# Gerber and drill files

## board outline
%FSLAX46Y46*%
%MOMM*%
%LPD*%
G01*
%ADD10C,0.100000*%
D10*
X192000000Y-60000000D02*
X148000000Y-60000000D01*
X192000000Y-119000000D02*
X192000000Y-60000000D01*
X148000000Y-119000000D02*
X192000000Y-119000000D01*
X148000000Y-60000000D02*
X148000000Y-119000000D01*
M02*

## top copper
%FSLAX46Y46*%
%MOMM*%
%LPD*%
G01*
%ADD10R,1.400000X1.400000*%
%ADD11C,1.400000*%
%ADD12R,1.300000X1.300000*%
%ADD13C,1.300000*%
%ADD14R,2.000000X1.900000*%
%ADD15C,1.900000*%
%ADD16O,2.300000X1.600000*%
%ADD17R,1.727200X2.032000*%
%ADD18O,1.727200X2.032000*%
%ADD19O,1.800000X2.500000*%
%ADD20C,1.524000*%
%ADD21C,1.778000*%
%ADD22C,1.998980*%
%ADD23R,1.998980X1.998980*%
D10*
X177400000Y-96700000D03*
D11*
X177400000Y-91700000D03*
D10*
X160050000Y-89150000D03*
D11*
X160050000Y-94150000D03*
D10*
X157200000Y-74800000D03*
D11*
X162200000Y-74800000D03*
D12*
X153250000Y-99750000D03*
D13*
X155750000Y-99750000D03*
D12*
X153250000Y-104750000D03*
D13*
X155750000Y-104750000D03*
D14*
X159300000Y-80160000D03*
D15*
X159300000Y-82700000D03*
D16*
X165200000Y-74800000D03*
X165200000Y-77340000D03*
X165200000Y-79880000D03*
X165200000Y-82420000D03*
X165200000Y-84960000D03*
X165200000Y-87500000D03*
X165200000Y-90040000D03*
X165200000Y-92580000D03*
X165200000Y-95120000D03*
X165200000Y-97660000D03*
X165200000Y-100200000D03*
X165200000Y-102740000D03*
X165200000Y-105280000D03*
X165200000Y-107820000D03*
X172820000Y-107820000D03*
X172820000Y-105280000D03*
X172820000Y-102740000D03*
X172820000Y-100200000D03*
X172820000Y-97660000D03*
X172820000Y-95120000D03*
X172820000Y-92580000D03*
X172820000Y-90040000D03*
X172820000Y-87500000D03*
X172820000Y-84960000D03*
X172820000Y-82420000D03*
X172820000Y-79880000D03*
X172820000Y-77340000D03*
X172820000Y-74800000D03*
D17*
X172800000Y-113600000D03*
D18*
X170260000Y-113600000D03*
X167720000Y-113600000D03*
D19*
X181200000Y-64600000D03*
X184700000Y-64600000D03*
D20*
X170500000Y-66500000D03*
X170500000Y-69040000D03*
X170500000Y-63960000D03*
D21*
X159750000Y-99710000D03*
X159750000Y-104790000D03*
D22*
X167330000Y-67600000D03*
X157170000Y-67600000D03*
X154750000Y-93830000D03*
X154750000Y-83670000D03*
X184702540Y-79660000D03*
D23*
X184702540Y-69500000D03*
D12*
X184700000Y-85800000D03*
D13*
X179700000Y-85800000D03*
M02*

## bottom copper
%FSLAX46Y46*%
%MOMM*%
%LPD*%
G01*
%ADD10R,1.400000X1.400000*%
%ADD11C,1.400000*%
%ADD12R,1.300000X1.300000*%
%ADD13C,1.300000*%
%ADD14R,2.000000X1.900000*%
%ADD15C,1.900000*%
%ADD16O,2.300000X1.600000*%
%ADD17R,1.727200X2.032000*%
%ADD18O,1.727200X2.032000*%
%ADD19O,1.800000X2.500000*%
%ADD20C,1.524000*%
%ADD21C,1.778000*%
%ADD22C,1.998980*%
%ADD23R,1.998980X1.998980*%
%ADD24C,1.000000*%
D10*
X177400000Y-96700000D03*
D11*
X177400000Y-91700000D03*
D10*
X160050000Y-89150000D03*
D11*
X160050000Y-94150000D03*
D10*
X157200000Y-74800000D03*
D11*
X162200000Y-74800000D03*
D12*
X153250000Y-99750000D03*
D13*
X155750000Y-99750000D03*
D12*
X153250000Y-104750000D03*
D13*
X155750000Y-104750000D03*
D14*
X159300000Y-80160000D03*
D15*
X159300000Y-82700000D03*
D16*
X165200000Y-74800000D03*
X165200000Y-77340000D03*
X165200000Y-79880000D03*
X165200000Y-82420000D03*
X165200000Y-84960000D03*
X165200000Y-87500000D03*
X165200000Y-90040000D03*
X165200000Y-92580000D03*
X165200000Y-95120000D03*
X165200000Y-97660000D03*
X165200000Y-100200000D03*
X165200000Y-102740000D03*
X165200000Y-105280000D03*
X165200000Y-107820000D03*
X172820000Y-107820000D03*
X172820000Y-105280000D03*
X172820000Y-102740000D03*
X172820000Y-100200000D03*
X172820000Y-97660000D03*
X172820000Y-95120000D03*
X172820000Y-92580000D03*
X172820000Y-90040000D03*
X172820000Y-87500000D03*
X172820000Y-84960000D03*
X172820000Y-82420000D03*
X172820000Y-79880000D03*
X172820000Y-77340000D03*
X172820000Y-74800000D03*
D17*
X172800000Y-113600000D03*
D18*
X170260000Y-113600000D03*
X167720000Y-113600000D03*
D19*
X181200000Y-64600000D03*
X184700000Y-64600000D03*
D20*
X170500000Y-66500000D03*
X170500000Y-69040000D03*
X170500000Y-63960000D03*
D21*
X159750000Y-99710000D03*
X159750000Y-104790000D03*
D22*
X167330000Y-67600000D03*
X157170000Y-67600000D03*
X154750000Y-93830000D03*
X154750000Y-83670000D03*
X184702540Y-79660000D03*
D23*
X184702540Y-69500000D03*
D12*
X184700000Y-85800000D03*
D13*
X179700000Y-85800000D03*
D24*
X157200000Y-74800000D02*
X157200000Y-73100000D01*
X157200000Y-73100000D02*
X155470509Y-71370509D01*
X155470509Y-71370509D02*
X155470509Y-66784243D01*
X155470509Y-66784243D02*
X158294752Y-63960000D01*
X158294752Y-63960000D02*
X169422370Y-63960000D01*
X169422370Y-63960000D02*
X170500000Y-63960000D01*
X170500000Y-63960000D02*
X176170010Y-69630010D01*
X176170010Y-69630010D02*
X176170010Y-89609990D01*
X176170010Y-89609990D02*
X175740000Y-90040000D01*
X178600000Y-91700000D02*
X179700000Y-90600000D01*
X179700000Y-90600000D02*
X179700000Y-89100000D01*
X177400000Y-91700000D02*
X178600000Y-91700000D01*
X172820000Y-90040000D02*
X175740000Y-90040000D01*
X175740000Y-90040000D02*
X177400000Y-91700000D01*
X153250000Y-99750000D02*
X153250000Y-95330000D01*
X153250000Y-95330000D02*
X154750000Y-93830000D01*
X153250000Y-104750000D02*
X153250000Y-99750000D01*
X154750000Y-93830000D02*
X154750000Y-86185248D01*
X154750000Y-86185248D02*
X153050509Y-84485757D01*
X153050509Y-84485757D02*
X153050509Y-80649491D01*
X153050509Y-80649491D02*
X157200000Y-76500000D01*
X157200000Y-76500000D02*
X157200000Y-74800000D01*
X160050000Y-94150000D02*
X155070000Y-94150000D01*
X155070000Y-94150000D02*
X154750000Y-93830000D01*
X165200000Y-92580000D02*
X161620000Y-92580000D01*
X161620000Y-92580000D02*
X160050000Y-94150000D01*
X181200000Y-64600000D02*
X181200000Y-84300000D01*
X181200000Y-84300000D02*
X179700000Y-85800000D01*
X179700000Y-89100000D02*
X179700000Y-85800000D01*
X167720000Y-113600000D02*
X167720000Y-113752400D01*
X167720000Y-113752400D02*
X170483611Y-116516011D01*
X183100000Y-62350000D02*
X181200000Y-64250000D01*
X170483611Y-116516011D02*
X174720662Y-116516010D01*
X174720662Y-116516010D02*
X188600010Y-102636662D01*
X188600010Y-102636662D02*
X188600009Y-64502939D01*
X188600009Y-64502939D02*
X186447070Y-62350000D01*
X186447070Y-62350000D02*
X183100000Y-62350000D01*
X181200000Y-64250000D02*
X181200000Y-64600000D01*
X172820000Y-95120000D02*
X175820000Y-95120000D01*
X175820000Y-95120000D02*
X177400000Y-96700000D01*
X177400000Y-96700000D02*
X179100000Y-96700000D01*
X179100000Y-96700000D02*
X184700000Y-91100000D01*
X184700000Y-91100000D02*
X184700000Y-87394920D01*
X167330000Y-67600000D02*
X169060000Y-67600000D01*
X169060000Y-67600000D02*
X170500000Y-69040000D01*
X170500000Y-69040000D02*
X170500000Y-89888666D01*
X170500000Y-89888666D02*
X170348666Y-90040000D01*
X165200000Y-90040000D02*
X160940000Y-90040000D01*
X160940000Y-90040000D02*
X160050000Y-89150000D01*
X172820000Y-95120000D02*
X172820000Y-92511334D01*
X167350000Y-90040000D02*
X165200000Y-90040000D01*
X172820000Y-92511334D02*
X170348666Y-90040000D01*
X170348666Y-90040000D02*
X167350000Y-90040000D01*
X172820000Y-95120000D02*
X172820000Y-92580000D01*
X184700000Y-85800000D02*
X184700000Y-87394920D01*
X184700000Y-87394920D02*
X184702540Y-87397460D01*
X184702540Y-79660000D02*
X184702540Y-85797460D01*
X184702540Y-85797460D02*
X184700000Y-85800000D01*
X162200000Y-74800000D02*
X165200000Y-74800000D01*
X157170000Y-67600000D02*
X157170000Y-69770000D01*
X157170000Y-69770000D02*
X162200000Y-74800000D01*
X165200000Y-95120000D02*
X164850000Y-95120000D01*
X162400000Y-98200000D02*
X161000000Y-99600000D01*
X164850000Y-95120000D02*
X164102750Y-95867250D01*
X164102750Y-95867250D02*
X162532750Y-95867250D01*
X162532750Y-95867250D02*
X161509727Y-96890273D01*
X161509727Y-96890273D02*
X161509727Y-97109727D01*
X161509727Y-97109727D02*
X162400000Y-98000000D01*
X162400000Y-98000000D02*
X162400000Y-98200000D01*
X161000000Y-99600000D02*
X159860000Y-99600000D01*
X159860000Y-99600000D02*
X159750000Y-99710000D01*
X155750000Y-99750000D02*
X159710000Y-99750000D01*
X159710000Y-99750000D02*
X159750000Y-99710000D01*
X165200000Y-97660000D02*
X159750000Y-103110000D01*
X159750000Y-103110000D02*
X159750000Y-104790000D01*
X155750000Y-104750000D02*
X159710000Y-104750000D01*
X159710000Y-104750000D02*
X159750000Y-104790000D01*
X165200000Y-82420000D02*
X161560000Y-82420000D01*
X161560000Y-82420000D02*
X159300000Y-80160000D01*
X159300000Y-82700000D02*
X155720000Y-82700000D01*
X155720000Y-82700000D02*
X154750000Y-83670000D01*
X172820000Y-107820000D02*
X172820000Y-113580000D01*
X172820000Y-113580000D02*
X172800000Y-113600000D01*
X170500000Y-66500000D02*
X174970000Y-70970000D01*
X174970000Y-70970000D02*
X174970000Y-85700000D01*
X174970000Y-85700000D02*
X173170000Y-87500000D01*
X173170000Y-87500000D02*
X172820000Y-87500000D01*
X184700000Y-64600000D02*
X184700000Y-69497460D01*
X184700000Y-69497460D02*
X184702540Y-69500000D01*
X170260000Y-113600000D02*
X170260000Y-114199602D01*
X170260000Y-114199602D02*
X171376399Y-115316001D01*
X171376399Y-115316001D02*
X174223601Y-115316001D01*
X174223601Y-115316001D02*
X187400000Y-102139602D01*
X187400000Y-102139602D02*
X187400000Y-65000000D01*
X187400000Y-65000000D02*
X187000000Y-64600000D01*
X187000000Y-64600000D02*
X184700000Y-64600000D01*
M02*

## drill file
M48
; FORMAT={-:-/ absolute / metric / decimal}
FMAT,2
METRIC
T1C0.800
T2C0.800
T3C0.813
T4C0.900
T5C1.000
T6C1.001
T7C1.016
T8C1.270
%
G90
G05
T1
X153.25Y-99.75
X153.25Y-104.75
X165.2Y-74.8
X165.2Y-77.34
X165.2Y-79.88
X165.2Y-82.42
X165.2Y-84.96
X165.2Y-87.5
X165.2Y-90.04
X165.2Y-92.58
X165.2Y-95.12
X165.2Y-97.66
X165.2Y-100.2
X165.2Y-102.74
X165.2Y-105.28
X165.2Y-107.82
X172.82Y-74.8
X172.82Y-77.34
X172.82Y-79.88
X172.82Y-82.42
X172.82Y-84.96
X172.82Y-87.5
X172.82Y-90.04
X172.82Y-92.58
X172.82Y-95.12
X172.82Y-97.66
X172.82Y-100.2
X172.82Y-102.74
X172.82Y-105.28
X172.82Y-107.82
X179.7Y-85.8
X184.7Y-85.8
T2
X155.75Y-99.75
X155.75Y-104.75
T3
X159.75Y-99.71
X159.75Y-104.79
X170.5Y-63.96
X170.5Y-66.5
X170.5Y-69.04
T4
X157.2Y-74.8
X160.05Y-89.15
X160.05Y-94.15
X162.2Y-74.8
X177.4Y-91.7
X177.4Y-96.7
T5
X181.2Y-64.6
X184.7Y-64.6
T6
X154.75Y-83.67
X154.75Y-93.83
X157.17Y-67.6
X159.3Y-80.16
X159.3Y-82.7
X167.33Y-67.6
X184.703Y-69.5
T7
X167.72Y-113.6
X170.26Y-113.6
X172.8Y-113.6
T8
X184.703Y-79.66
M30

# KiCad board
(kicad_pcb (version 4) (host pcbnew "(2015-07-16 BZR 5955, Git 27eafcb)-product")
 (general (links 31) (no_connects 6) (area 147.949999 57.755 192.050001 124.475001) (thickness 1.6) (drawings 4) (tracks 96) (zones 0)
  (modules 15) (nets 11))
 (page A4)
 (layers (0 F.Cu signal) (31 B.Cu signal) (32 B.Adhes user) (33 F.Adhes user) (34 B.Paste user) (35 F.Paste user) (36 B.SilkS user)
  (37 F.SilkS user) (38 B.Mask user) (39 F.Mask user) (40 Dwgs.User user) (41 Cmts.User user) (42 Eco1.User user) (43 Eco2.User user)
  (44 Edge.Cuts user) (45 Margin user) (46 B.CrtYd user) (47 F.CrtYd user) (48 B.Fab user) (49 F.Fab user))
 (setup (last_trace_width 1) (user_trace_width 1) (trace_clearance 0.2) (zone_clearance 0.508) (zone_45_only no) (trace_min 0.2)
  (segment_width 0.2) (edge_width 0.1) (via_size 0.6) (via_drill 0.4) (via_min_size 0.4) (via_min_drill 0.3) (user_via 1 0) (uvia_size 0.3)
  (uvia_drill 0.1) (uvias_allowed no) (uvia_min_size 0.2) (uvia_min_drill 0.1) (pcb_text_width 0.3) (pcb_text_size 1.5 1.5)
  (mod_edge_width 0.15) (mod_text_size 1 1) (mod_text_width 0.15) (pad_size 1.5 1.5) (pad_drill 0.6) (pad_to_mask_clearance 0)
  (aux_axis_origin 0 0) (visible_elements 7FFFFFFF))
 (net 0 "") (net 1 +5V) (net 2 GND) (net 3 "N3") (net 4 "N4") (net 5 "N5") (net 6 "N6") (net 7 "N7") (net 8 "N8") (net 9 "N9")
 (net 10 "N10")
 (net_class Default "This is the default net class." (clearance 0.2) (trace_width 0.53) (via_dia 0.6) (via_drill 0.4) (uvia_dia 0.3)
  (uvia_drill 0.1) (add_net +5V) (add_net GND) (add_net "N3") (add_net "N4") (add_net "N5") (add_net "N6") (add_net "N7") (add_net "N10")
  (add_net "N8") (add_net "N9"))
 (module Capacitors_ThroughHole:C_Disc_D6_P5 (layer F.Cu) (at 177.4 96.7 90)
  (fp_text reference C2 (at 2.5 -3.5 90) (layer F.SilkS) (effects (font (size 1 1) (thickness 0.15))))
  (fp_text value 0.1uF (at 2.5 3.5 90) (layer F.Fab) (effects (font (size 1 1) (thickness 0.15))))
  (pad 1 thru_hole rect (at 0 0 90) (size 1.4 1.4) (drill 0.9) (layers *.Cu *.Mask F.SilkS) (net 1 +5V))
  (pad 2 thru_hole circle (at 5 0 90) (size 1.4 1.4) (drill 0.9) (layers *.Cu *.Mask F.SilkS) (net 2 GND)))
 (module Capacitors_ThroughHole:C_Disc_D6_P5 (layer F.Cu) (at 160.05 89.15 270)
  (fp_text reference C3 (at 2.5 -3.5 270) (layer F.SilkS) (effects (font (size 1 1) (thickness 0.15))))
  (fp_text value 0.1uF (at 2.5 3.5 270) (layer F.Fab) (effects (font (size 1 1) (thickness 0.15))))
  (pad 1 thru_hole rect (at 0 0 270) (size 1.4 1.4) (drill 0.9) (layers *.Cu *.Mask F.SilkS) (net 1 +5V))
  (pad 2 thru_hole circle (at 5 0 270) (size 1.4 1.4) (drill 0.9) (layers *.Cu *.Mask F.SilkS) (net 2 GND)))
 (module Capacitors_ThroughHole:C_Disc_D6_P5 (layer F.Cu) (at 157.2 74.8)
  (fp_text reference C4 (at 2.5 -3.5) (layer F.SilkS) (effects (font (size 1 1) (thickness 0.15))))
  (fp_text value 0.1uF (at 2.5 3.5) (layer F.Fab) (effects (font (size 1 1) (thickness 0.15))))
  (pad 1 thru_hole rect (at 0 0) (size 1.4 1.4) (drill 0.9) (layers *.Cu *.Mask F.SilkS) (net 2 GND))
  (pad 2 thru_hole circle (at 5 0) (size 1.4 1.4) (drill 0.9) (layers *.Cu *.Mask F.SilkS) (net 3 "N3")))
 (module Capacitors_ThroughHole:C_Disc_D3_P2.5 (layer F.Cu) (at 153.25 99.75)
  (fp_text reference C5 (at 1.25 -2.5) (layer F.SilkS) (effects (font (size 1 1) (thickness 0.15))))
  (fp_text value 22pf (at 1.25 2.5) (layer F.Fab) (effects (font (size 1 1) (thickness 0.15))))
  (pad 1 thru_hole rect (at 0 0) (size 1.3 1.3) (drill 0.8) (layers *.Cu *.Mask F.SilkS) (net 2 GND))
  (pad 2 thru_hole circle (at 2.5 0) (size 1.3 1.3) (drill 0.8001) (layers *.Cu *.Mask F.SilkS) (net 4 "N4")))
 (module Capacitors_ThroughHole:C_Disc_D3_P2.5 (layer F.Cu) (at 153.25 104.75)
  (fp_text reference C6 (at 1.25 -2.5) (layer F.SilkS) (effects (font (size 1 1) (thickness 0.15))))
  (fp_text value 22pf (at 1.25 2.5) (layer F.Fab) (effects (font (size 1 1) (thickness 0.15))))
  (pad 1 thru_hole rect (at 0 0) (size 1.3 1.3) (drill 0.8) (layers *.Cu *.Mask F.SilkS) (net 2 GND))
  (pad 2 thru_hole circle (at 2.5 0) (size 1.3 1.3) (drill 0.8001) (layers *.Cu *.Mask F.SilkS) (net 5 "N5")))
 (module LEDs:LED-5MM (layer F.Cu) (at 159.3 80.16 270)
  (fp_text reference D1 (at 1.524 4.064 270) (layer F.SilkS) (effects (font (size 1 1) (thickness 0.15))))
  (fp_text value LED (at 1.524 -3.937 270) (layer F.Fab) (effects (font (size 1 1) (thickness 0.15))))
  (pad 1 thru_hole rect (at 0 0) (size 2 1.9) (drill 1.00076) (layers *.Cu *.Mask F.SilkS) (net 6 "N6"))
  (pad 2 thru_hole circle (at 2.54 0 270) (size 1.9 1.9) (drill 1.00076) (layers *.Cu *.Mask F.SilkS) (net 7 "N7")))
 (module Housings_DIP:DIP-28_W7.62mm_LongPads (layer F.Cu) (at 165.2 74.8)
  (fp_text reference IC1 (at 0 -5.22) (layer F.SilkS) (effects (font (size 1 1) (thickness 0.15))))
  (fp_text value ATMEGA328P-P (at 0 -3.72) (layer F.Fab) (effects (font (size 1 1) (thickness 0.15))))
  (pad 1 thru_hole oval (at 0 0) (size 2.3 1.6) (drill 0.8) (layers *.Cu *.Mask F.SilkS) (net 3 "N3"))
  (pad 2 thru_hole oval (at 0 2.54) (size 2.3 1.6) (drill 0.8) (layers *.Cu *.Mask F.SilkS))
  (pad 3 thru_hole oval (at 0 5.08) (size 2.3 1.6) (drill 0.8) (layers *.Cu *.Mask F.SilkS))
  (pad 4 thru_hole oval (at 0 7.62) (size 2.3 1.6) (drill 0.8) (layers *.Cu *.Mask F.SilkS) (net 6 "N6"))
  (pad 5 thru_hole oval (at 0 10.16) (size 2.3 1.6) (drill 0.8) (layers *.Cu *.Mask F.SilkS))
  (pad 6 thru_hole oval (at 0 12.7) (size 2.3 1.6) (drill 0.8) (layers *.Cu *.Mask F.SilkS))
  (pad 7 thru_hole oval (at 0 15.24) (size 2.3 1.6) (drill 0.8) (layers *.Cu *.Mask F.SilkS) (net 1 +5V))
  (pad 8 thru_hole oval (at 0 17.78) (size 2.3 1.6) (drill 0.8) (layers *.Cu *.Mask F.SilkS) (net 2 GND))
  (pad 9 thru_hole oval (at 0 20.32) (size 2.3 1.6) (drill 0.8) (layers *.Cu *.Mask F.SilkS) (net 4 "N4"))
  (pad 10 thru_hole oval (at 0 22.86) (size 2.3 1.6) (drill 0.8) (layers *.Cu *.Mask F.SilkS) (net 5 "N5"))
  (pad 11 thru_hole oval (at 0 25.4) (size 2.3 1.6) (drill 0.8) (layers *.Cu *.Mask F.SilkS))
  (pad 12 thru_hole oval (at 0 27.94) (size 2.3 1.6) (drill 0.8) (layers *.Cu *.Mask F.SilkS))
  (pad 13 thru_hole oval (at 0 30.48) (size 2.3 1.6) (drill 0.8) (layers *.Cu *.Mask F.SilkS))
  (pad 14 thru_hole oval (at 0 33.02) (size 2.3 1.6) (drill 0.8) (layers *.Cu *.Mask F.SilkS))
  (pad 15 thru_hole oval (at 7.62 33.02) (size 2.3 1.6) (drill 0.8) (layers *.Cu *.Mask F.SilkS) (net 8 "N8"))
  (pad 16 thru_hole oval (at 7.62 30.48) (size 2.3 1.6) (drill 0.8) (layers *.Cu *.Mask F.SilkS))
  (pad 17 thru_hole oval (at 7.62 27.94) (size 2.3 1.6) (drill 0.8) (layers *.Cu *.Mask F.SilkS))
  (pad 18 thru_hole oval (at 7.62 25.4) (size 2.3 1.6) (drill 0.8) (layers *.Cu *.Mask F.SilkS))
  (pad 19 thru_hole oval (at 7.62 22.86) (size 2.3 1.6) (drill 0.8) (layers *.Cu *.Mask F.SilkS))
  (pad 20 thru_hole oval (at 7.62 20.32) (size 2.3 1.6) (drill 0.8) (layers *.Cu *.Mask F.SilkS) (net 1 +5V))
  (pad 21 thru_hole oval (at 7.62 17.78) (size 2.3 1.6) (drill 0.8) (layers *.Cu *.Mask F.SilkS) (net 1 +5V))
  (pad 22 thru_hole oval (at 7.62 15.24) (size 2.3 1.6) (drill 0.8) (layers *.Cu *.Mask F.SilkS) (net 2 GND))
  (pad 23 thru_hole oval (at 7.62 12.7) (size 2.3 1.6) (drill 0.8) (layers *.Cu *.Mask F.SilkS) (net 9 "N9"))
  (pad 24 thru_hole oval (at 7.62 10.16) (size 2.3 1.6) (drill 0.8) (layers *.Cu *.Mask F.SilkS))
  (pad 25 thru_hole oval (at 7.62 7.62) (size 2.3 1.6) (drill 0.8) (layers *.Cu *.Mask F.SilkS))
  (pad 26 thru_hole oval (at 7.62 5.08) (size 2.3 1.6) (drill 0.8) (layers *.Cu *.Mask F.SilkS))
  (pad 27 thru_hole oval (at 7.62 2.54) (size 2.3 1.6) (drill 0.8) (layers *.Cu *.Mask F.SilkS))
  (pad 28 thru_hole oval (at 7.62 0) (size 2.3 1.6) (drill 0.8) (layers *.Cu *.Mask F.SilkS)))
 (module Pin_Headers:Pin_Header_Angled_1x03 (layer F.Cu) (at 172.8 113.6 270)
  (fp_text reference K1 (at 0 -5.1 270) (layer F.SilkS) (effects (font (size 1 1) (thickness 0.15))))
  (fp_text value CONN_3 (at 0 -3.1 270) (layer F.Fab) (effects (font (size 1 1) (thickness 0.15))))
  (pad 1 thru_hole rect (at 0 0 270) (size 2.032 1.7272) (drill 1.016) (layers *.Cu *.Mask F.SilkS) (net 8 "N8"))
  (pad 2 thru_hole oval (at 0 2.54 270) (size 2.032 1.7272) (drill 1.016) (layers *.Cu *.Mask F.SilkS) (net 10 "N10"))
  (pad 3 thru_hole oval (at 0 5.08 270) (size 2.032 1.7272) (drill 1.016) (layers *.Cu *.Mask F.SilkS) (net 2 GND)))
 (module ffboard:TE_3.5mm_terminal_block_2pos (layer F.Cu) (at 181.2 64.6)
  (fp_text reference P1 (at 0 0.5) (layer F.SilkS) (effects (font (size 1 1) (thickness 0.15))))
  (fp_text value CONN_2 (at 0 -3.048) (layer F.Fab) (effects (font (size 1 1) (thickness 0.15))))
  (pad 1 thru_hole oval (at 0 0) (size 1.8 2.5) (drill 1) (layers *.Cu *.Mask F.SilkS) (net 2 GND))
  (pad 2 thru_hole oval (at 3.5 0) (size 1.8 2.5) (drill 1) (layers *.Cu *.Mask F.SilkS) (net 10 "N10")))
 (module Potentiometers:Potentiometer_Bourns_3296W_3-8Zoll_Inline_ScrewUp (layer F.Cu) (at 170.5 63.96 180)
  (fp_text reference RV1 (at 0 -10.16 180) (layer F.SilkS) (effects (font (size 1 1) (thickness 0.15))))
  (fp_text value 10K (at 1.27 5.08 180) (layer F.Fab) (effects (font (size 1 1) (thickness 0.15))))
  (pad 2 thru_hole circle (at 0 -2.54 180) (size 1.524 1.524) (drill 0.8128) (layers *.Cu *.Mask F.SilkS) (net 9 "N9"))
  (pad 3 thru_hole circle (at 0 -5.08 180) (size 1.524 1.524) (drill 0.8128) (layers *.Cu *.Mask F.SilkS) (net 1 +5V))
  (pad 1 thru_hole circle (at 0 0 180) (size 1.524 1.524) (drill 0.8128) (layers *.Cu *.Mask F.SilkS) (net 2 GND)))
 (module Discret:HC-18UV (layer F.Cu) (at 159.75 102.25 270)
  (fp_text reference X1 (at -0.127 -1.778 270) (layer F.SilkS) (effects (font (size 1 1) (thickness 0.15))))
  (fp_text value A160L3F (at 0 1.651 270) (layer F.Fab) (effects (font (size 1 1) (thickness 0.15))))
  (pad 1 thru_hole circle (at -2.54 0 270) (size 1.778 1.778) (drill 0.8128) (layers *.Cu *.Mask F.SilkS) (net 4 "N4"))
  (pad 2 thru_hole circle (at 2.54 0 270) (size 1.778 1.778) (drill 0.8128) (layers *.Cu *.Mask F.SilkS) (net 5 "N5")))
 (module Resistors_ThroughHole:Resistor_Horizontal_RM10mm (layer F.Cu) (at 162.25 67.6 180)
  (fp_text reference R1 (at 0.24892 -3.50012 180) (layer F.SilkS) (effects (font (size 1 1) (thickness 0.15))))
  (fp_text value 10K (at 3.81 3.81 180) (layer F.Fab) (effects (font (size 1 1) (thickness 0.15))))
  (pad 1 thru_hole circle (at -5.08 0 180) (size 1.99898 1.99898) (drill 1.00076) (layers *.Cu *.SilkS *.Mask) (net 1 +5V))
  (pad 2 thru_hole circle (at 5.08 0 180) (size 1.99898 1.99898) (drill 1.00076) (layers *.Cu *.SilkS *.Mask) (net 3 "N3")))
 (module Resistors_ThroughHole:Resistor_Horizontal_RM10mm (layer F.Cu) (at 154.75 88.75 90)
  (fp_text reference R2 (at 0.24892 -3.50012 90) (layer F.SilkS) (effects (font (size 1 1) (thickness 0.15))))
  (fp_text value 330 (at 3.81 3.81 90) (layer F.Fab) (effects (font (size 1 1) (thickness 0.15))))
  (pad 1 thru_hole circle (at -5.08 0 90) (size 1.99898 1.99898) (drill 1.00076) (layers *.Cu *.SilkS *.Mask) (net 2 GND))
  (pad 2 thru_hole circle (at 5.08 0 90) (size 1.99898 1.99898) (drill 1.00076) (layers *.Cu *.SilkS *.Mask) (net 7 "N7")))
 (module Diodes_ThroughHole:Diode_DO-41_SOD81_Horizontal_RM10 (layer F.Cu) (at 184.7 69.5 270)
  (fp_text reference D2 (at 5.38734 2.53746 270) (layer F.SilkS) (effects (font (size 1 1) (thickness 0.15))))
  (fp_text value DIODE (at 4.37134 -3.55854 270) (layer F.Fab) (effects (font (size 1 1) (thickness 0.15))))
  (pad 2 thru_hole circle (at 10.16 -0.00254 90) (size 1.99898 1.99898) (drill 1.27) (layers *.Cu *.Mask F.SilkS) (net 1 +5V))
  (pad 1 thru_hole rect (at 0 -0.00254 90) (size 1.99898 1.99898) (drill 1.00076) (layers *.Cu *.Mask F.SilkS) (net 10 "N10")))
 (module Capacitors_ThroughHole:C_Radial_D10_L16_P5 (layer F.Cu) (at 184.7 85.8 180)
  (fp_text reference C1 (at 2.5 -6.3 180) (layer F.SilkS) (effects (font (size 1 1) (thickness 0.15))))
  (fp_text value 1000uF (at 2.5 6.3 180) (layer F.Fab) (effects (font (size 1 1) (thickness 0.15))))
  (pad 1 thru_hole rect (at 0 0 180) (size 1.3 1.3) (drill 0.8) (layers *.Cu *.Mask F.SilkS) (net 1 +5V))
  (pad 2 thru_hole circle (at 5 0 180) (size 1.3 1.3) (drill 0.8) (layers *.Cu *.Mask F.SilkS) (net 2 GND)))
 (gr_line (start 192 60) (end 148 60) (layer Edge.Cuts) (width 0.1))
 (gr_line (start 192 119) (end 192 60) (layer Edge.Cuts) (width 0.1))
 (gr_line (start 148 119) (end 192 119) (layer Edge.Cuts) (width 0.1))
 (gr_line (start 148 60) (end 148 119) (layer Edge.Cuts) (width 0.1))
 (segment (start 157.2 74.8) (end 157.2 73.1) (width 1) (layer B.Cu) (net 2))
 (segment (start 157.2 73.1) (end 155.470509 71.370509) (width 1) (layer B.Cu) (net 2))
 (segment (start 155.470509 71.370509) (end 155.470509 66.784243) (width 1) (layer B.Cu) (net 2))
 (segment (start 155.470509 66.784243) (end 158.294752 63.96) (width 1) (layer B.Cu) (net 2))
 (segment (start 158.294752 63.96) (end 169.42237 63.96) (width 1) (layer B.Cu) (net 2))
 (segment (start 169.42237 63.96) (end 170.5 63.96) (width 1) (layer B.Cu) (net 2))
 (segment (start 170.5 63.96) (end 176.17001 69.63001) (width 1) (layer B.Cu) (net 2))
 (segment (start 176.17001 69.63001) (end 176.17001 89.60999) (width 1) (layer B.Cu) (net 2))
 (segment (start 176.17001 89.60999) (end 175.74 90.04) (width 1) (layer B.Cu) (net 2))
 (segment (start 178.6 91.7) (end 179.7 90.6) (width 1) (layer B.Cu) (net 2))
 (segment (start 179.7 90.6) (end 179.7 89.1) (width 1) (layer B.Cu) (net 2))
 (segment (start 177.4 91.7) (end 178.6 91.7) (width 1) (layer B.Cu) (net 2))
 (segment (start 172.82 90.04) (end 175.74 90.04) (width 1) (layer B.Cu) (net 2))
 (segment (start 175.74 90.04) (end 177.4 91.7) (width 1) (layer B.Cu) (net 2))
 (segment (start 153.25 99.75) (end 153.25 95.33) (width 1) (layer B.Cu) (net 2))
 (segment (start 153.25 95.33) (end 154.75 93.83) (width 1) (layer B.Cu) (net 2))
 (segment (start 153.25 104.75) (end 153.25 99.75) (width 1) (layer B.Cu) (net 2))
 (segment (start 154.75 93.83) (end 154.75 86.185248) (width 1) (layer B.Cu) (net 2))
 (segment (start 154.75 86.185248) (end 153.050509 84.485757) (width 1) (layer B.Cu) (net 2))
 (segment (start 153.050509 84.485757) (end 153.050509 80.649491) (width 1) (layer B.Cu) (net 2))
 (segment (start 153.050509 80.649491) (end 157.2 76.5) (width 1) (layer B.Cu) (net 2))
 (segment (start 157.2 76.5) (end 157.2 74.8) (width 1) (layer B.Cu) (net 2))
 (segment (start 160.05 94.15) (end 155.07 94.15) (width 1) (layer B.Cu) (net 2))
 (segment (start 155.07 94.15) (end 154.75 93.83) (width 1) (layer B.Cu) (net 2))
 (segment (start 165.2 92.58) (end 161.62 92.58) (width 1) (layer B.Cu) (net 2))
 (segment (start 161.62 92.58) (end 160.05 94.15) (width 1) (layer B.Cu) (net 2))
 (segment (start 181.2 64.6) (end 181.2 84.3) (width 1) (layer B.Cu) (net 2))
 (segment (start 181.2 84.3) (end 179.7 85.8) (width 1) (layer B.Cu) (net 2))
 (segment (start 179.7 89.1) (end 179.7 85.8) (width 1) (layer B.Cu) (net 2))
 (segment (start 167.72 113.6) (end 167.72 113.7524) (width 1) (layer B.Cu) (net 2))
 (segment (start 167.72 113.7524) (end 170.483611 116.516011) (width 1) (layer B.Cu) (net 2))
 (segment (start 183.1 62.35) (end 181.2 64.25) (width 1) (layer B.Cu) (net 2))
 (segment (start 170.483611 116.516011) (end 174.720662 116.51601) (width 1) (layer B.Cu) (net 2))
 (segment (start 174.720662 116.51601) (end 188.60001 102.636662) (width 1) (layer B.Cu) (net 2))
 (segment (start 188.60001 102.636662) (end 188.600009 64.502939) (width 1) (layer B.Cu) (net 2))
 (segment (start 188.600009 64.502939) (end 186.44707 62.35) (width 1) (layer B.Cu) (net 2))
 (segment (start 186.44707 62.35) (end 183.1 62.35) (width 1) (layer B.Cu) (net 2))
 (segment (start 181.2 64.25) (end 181.2 64.6) (width 1) (layer B.Cu) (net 2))
 (segment (start 172.82 95.12) (end 175.82 95.12) (width 1) (layer B.Cu) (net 1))
 (segment (start 175.82 95.12) (end 177.4 96.7) (width 1) (layer B.Cu) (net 1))
 (segment (start 177.4 96.7) (end 179.1 96.7) (width 1) (layer B.Cu) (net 1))
 (segment (start 179.1 96.7) (end 184.7 91.1) (width 1) (layer B.Cu) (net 1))
 (segment (start 184.7 91.1) (end 184.7 87.39492) (width 1) (layer B.Cu) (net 1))
 (segment (start 167.33 67.6) (end 169.06 67.6) (width 1) (layer B.Cu) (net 1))
 (segment (start 169.06 67.6) (end 170.5 69.04) (width 1) (layer B.Cu) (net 1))
 (segment (start 170.5 69.04) (end 170.5 89.888666) (width 1) (layer B.Cu) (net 1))
 (segment (start 170.5 89.888666) (end 170.348666 90.04) (width 1) (layer B.Cu) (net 1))
 (segment (start 165.2 90.04) (end 160.94 90.04) (width 1) (layer B.Cu) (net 1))
 (segment (start 160.94 90.04) (end 160.05 89.15) (width 1) (layer B.Cu) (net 1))
 (segment (start 172.82 95.12) (end 172.82 92.511334) (width 1) (layer B.Cu) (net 1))
 (segment (start 167.35 90.04) (end 165.2 90.04) (width 1) (layer B.Cu) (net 1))
 (segment (start 172.82 92.511334) (end 170.348666 90.04) (width 1) (layer B.Cu) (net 1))
 (segment (start 170.348666 90.04) (end 167.35 90.04) (width 1) (layer B.Cu) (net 1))
 (segment (start 172.82 95.12) (end 172.82 92.58) (width 1) (layer B.Cu) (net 1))
 (segment (start 184.7 85.8) (end 184.7 87.39492) (width 1) (layer B.Cu) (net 1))
 (segment (start 184.7 87.39492) (end 184.70254 87.39746) (width 1) (layer B.Cu) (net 1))
 (segment (start 184.70254 79.66) (end 184.70254 85.79746) (width 1) (layer B.Cu) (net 1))
 (segment (start 184.70254 85.79746) (end 184.7 85.8) (width 1) (layer B.Cu) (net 1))
 (segment (start 162.2 74.8) (end 165.2 74.8) (width 1) (layer B.Cu) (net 3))
 (segment (start 157.17 67.6) (end 157.17 69.77) (width 1) (layer B.Cu) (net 3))
 (segment (start 157.17 69.77) (end 162.2 74.8) (width 1) (layer B.Cu) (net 3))
 (segment (start 165.2 95.12) (end 164.85 95.12) (width 1) (layer B.Cu) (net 4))
 (segment (start 162.4 98.2) (end 161 99.6) (width 1) (layer B.Cu) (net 4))
 (segment (start 164.85 95.12) (end 164.10275 95.86725) (width 1) (layer B.Cu) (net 4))
 (segment (start 164.10275 95.86725) (end 162.53275 95.86725) (width 1) (layer B.Cu) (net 4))
 (segment (start 162.53275 95.86725) (end 161.509727 96.890273) (width 1) (layer B.Cu) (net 4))
 (segment (start 161.509727 96.890273) (end 161.509727 97.109727) (width 1) (layer B.Cu) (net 4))
 (segment (start 161.509727 97.109727) (end 162.4 98) (width 1) (layer B.Cu) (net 4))
 (segment (start 162.4 98) (end 162.4 98.2) (width 1) (layer B.Cu) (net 4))
 (segment (start 161 99.6) (end 159.86 99.6) (width 1) (layer B.Cu) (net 4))
 (segment (start 159.86 99.6) (end 159.75 99.71) (width 1) (layer B.Cu) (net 4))
 (segment (start 155.75 99.75) (end 159.71 99.75) (width 1) (layer B.Cu) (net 4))
 (segment (start 159.71 99.75) (end 159.75 99.71) (width 1) (layer B.Cu) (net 4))
 (segment (start 165.2 97.66) (end 159.75 103.11) (width 1) (layer B.Cu) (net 5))
 (segment (start 159.75 103.11) (end 159.75 104.79) (width 1) (layer B.Cu) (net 5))
 (segment (start 155.75 104.75) (end 159.71 104.75) (width 1) (layer B.Cu) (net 5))
 (segment (start 159.71 104.75) (end 159.75 104.79) (width 1) (layer B.Cu) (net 5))
 (segment (start 165.2 82.42) (end 161.56 82.42) (width 1) (layer B.Cu) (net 6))
 (segment (start 161.56 82.42) (end 159.3 80.16) (width 1) (layer B.Cu) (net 6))
 (segment (start 159.3 82.7) (end 155.72 82.7) (width 1) (layer B.Cu) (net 7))
 (segment (start 155.72 82.7) (end 154.75 83.67) (width 1) (layer B.Cu) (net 7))
 (segment (start 172.82 107.82) (end 172.82 113.58) (width 1) (layer B.Cu) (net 8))
 (segment (start 172.82 113.58) (end 172.8 113.6) (width 1) (layer B.Cu) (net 8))
 (segment (start 170.5 66.5) (end 174.97 70.97) (width 1) (layer B.Cu) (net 9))
 (segment (start 174.97 70.97) (end 174.97 85.7) (width 1) (layer B.Cu) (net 9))
 (segment (start 174.97 85.7) (end 173.17 87.5) (width 1) (layer B.Cu) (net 9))
 (segment (start 173.17 87.5) (end 172.82 87.5) (width 1) (layer B.Cu) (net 9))
 (segment (start 184.7 64.6) (end 184.7 69.49746) (width 1) (layer B.Cu) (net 10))
 (segment (start 184.7 69.49746) (end 184.70254 69.5) (width 1) (layer B.Cu) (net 10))
 (segment (start 170.26 113.6) (end 170.26 114.199602) (width 1) (layer B.Cu) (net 10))
 (segment (start 170.26 114.199602) (end 171.376399 115.316001) (width 1) (layer B.Cu) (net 10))
 (segment (start 171.376399 115.316001) (end 174.223601 115.316001) (width 1) (layer B.Cu) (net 10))
 (segment (start 174.223601 115.316001) (end 187.4 102.139602) (width 1) (layer B.Cu) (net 10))
 (segment (start 187.4 102.139602) (end 187.4 65) (width 1) (layer B.Cu) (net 10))
 (segment (start 187.4 65) (end 187 64.6) (width 1) (layer B.Cu) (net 10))
 (segment (start 187 64.6) (end 184.7 64.6) (width 1) (layer B.Cu) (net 10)))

